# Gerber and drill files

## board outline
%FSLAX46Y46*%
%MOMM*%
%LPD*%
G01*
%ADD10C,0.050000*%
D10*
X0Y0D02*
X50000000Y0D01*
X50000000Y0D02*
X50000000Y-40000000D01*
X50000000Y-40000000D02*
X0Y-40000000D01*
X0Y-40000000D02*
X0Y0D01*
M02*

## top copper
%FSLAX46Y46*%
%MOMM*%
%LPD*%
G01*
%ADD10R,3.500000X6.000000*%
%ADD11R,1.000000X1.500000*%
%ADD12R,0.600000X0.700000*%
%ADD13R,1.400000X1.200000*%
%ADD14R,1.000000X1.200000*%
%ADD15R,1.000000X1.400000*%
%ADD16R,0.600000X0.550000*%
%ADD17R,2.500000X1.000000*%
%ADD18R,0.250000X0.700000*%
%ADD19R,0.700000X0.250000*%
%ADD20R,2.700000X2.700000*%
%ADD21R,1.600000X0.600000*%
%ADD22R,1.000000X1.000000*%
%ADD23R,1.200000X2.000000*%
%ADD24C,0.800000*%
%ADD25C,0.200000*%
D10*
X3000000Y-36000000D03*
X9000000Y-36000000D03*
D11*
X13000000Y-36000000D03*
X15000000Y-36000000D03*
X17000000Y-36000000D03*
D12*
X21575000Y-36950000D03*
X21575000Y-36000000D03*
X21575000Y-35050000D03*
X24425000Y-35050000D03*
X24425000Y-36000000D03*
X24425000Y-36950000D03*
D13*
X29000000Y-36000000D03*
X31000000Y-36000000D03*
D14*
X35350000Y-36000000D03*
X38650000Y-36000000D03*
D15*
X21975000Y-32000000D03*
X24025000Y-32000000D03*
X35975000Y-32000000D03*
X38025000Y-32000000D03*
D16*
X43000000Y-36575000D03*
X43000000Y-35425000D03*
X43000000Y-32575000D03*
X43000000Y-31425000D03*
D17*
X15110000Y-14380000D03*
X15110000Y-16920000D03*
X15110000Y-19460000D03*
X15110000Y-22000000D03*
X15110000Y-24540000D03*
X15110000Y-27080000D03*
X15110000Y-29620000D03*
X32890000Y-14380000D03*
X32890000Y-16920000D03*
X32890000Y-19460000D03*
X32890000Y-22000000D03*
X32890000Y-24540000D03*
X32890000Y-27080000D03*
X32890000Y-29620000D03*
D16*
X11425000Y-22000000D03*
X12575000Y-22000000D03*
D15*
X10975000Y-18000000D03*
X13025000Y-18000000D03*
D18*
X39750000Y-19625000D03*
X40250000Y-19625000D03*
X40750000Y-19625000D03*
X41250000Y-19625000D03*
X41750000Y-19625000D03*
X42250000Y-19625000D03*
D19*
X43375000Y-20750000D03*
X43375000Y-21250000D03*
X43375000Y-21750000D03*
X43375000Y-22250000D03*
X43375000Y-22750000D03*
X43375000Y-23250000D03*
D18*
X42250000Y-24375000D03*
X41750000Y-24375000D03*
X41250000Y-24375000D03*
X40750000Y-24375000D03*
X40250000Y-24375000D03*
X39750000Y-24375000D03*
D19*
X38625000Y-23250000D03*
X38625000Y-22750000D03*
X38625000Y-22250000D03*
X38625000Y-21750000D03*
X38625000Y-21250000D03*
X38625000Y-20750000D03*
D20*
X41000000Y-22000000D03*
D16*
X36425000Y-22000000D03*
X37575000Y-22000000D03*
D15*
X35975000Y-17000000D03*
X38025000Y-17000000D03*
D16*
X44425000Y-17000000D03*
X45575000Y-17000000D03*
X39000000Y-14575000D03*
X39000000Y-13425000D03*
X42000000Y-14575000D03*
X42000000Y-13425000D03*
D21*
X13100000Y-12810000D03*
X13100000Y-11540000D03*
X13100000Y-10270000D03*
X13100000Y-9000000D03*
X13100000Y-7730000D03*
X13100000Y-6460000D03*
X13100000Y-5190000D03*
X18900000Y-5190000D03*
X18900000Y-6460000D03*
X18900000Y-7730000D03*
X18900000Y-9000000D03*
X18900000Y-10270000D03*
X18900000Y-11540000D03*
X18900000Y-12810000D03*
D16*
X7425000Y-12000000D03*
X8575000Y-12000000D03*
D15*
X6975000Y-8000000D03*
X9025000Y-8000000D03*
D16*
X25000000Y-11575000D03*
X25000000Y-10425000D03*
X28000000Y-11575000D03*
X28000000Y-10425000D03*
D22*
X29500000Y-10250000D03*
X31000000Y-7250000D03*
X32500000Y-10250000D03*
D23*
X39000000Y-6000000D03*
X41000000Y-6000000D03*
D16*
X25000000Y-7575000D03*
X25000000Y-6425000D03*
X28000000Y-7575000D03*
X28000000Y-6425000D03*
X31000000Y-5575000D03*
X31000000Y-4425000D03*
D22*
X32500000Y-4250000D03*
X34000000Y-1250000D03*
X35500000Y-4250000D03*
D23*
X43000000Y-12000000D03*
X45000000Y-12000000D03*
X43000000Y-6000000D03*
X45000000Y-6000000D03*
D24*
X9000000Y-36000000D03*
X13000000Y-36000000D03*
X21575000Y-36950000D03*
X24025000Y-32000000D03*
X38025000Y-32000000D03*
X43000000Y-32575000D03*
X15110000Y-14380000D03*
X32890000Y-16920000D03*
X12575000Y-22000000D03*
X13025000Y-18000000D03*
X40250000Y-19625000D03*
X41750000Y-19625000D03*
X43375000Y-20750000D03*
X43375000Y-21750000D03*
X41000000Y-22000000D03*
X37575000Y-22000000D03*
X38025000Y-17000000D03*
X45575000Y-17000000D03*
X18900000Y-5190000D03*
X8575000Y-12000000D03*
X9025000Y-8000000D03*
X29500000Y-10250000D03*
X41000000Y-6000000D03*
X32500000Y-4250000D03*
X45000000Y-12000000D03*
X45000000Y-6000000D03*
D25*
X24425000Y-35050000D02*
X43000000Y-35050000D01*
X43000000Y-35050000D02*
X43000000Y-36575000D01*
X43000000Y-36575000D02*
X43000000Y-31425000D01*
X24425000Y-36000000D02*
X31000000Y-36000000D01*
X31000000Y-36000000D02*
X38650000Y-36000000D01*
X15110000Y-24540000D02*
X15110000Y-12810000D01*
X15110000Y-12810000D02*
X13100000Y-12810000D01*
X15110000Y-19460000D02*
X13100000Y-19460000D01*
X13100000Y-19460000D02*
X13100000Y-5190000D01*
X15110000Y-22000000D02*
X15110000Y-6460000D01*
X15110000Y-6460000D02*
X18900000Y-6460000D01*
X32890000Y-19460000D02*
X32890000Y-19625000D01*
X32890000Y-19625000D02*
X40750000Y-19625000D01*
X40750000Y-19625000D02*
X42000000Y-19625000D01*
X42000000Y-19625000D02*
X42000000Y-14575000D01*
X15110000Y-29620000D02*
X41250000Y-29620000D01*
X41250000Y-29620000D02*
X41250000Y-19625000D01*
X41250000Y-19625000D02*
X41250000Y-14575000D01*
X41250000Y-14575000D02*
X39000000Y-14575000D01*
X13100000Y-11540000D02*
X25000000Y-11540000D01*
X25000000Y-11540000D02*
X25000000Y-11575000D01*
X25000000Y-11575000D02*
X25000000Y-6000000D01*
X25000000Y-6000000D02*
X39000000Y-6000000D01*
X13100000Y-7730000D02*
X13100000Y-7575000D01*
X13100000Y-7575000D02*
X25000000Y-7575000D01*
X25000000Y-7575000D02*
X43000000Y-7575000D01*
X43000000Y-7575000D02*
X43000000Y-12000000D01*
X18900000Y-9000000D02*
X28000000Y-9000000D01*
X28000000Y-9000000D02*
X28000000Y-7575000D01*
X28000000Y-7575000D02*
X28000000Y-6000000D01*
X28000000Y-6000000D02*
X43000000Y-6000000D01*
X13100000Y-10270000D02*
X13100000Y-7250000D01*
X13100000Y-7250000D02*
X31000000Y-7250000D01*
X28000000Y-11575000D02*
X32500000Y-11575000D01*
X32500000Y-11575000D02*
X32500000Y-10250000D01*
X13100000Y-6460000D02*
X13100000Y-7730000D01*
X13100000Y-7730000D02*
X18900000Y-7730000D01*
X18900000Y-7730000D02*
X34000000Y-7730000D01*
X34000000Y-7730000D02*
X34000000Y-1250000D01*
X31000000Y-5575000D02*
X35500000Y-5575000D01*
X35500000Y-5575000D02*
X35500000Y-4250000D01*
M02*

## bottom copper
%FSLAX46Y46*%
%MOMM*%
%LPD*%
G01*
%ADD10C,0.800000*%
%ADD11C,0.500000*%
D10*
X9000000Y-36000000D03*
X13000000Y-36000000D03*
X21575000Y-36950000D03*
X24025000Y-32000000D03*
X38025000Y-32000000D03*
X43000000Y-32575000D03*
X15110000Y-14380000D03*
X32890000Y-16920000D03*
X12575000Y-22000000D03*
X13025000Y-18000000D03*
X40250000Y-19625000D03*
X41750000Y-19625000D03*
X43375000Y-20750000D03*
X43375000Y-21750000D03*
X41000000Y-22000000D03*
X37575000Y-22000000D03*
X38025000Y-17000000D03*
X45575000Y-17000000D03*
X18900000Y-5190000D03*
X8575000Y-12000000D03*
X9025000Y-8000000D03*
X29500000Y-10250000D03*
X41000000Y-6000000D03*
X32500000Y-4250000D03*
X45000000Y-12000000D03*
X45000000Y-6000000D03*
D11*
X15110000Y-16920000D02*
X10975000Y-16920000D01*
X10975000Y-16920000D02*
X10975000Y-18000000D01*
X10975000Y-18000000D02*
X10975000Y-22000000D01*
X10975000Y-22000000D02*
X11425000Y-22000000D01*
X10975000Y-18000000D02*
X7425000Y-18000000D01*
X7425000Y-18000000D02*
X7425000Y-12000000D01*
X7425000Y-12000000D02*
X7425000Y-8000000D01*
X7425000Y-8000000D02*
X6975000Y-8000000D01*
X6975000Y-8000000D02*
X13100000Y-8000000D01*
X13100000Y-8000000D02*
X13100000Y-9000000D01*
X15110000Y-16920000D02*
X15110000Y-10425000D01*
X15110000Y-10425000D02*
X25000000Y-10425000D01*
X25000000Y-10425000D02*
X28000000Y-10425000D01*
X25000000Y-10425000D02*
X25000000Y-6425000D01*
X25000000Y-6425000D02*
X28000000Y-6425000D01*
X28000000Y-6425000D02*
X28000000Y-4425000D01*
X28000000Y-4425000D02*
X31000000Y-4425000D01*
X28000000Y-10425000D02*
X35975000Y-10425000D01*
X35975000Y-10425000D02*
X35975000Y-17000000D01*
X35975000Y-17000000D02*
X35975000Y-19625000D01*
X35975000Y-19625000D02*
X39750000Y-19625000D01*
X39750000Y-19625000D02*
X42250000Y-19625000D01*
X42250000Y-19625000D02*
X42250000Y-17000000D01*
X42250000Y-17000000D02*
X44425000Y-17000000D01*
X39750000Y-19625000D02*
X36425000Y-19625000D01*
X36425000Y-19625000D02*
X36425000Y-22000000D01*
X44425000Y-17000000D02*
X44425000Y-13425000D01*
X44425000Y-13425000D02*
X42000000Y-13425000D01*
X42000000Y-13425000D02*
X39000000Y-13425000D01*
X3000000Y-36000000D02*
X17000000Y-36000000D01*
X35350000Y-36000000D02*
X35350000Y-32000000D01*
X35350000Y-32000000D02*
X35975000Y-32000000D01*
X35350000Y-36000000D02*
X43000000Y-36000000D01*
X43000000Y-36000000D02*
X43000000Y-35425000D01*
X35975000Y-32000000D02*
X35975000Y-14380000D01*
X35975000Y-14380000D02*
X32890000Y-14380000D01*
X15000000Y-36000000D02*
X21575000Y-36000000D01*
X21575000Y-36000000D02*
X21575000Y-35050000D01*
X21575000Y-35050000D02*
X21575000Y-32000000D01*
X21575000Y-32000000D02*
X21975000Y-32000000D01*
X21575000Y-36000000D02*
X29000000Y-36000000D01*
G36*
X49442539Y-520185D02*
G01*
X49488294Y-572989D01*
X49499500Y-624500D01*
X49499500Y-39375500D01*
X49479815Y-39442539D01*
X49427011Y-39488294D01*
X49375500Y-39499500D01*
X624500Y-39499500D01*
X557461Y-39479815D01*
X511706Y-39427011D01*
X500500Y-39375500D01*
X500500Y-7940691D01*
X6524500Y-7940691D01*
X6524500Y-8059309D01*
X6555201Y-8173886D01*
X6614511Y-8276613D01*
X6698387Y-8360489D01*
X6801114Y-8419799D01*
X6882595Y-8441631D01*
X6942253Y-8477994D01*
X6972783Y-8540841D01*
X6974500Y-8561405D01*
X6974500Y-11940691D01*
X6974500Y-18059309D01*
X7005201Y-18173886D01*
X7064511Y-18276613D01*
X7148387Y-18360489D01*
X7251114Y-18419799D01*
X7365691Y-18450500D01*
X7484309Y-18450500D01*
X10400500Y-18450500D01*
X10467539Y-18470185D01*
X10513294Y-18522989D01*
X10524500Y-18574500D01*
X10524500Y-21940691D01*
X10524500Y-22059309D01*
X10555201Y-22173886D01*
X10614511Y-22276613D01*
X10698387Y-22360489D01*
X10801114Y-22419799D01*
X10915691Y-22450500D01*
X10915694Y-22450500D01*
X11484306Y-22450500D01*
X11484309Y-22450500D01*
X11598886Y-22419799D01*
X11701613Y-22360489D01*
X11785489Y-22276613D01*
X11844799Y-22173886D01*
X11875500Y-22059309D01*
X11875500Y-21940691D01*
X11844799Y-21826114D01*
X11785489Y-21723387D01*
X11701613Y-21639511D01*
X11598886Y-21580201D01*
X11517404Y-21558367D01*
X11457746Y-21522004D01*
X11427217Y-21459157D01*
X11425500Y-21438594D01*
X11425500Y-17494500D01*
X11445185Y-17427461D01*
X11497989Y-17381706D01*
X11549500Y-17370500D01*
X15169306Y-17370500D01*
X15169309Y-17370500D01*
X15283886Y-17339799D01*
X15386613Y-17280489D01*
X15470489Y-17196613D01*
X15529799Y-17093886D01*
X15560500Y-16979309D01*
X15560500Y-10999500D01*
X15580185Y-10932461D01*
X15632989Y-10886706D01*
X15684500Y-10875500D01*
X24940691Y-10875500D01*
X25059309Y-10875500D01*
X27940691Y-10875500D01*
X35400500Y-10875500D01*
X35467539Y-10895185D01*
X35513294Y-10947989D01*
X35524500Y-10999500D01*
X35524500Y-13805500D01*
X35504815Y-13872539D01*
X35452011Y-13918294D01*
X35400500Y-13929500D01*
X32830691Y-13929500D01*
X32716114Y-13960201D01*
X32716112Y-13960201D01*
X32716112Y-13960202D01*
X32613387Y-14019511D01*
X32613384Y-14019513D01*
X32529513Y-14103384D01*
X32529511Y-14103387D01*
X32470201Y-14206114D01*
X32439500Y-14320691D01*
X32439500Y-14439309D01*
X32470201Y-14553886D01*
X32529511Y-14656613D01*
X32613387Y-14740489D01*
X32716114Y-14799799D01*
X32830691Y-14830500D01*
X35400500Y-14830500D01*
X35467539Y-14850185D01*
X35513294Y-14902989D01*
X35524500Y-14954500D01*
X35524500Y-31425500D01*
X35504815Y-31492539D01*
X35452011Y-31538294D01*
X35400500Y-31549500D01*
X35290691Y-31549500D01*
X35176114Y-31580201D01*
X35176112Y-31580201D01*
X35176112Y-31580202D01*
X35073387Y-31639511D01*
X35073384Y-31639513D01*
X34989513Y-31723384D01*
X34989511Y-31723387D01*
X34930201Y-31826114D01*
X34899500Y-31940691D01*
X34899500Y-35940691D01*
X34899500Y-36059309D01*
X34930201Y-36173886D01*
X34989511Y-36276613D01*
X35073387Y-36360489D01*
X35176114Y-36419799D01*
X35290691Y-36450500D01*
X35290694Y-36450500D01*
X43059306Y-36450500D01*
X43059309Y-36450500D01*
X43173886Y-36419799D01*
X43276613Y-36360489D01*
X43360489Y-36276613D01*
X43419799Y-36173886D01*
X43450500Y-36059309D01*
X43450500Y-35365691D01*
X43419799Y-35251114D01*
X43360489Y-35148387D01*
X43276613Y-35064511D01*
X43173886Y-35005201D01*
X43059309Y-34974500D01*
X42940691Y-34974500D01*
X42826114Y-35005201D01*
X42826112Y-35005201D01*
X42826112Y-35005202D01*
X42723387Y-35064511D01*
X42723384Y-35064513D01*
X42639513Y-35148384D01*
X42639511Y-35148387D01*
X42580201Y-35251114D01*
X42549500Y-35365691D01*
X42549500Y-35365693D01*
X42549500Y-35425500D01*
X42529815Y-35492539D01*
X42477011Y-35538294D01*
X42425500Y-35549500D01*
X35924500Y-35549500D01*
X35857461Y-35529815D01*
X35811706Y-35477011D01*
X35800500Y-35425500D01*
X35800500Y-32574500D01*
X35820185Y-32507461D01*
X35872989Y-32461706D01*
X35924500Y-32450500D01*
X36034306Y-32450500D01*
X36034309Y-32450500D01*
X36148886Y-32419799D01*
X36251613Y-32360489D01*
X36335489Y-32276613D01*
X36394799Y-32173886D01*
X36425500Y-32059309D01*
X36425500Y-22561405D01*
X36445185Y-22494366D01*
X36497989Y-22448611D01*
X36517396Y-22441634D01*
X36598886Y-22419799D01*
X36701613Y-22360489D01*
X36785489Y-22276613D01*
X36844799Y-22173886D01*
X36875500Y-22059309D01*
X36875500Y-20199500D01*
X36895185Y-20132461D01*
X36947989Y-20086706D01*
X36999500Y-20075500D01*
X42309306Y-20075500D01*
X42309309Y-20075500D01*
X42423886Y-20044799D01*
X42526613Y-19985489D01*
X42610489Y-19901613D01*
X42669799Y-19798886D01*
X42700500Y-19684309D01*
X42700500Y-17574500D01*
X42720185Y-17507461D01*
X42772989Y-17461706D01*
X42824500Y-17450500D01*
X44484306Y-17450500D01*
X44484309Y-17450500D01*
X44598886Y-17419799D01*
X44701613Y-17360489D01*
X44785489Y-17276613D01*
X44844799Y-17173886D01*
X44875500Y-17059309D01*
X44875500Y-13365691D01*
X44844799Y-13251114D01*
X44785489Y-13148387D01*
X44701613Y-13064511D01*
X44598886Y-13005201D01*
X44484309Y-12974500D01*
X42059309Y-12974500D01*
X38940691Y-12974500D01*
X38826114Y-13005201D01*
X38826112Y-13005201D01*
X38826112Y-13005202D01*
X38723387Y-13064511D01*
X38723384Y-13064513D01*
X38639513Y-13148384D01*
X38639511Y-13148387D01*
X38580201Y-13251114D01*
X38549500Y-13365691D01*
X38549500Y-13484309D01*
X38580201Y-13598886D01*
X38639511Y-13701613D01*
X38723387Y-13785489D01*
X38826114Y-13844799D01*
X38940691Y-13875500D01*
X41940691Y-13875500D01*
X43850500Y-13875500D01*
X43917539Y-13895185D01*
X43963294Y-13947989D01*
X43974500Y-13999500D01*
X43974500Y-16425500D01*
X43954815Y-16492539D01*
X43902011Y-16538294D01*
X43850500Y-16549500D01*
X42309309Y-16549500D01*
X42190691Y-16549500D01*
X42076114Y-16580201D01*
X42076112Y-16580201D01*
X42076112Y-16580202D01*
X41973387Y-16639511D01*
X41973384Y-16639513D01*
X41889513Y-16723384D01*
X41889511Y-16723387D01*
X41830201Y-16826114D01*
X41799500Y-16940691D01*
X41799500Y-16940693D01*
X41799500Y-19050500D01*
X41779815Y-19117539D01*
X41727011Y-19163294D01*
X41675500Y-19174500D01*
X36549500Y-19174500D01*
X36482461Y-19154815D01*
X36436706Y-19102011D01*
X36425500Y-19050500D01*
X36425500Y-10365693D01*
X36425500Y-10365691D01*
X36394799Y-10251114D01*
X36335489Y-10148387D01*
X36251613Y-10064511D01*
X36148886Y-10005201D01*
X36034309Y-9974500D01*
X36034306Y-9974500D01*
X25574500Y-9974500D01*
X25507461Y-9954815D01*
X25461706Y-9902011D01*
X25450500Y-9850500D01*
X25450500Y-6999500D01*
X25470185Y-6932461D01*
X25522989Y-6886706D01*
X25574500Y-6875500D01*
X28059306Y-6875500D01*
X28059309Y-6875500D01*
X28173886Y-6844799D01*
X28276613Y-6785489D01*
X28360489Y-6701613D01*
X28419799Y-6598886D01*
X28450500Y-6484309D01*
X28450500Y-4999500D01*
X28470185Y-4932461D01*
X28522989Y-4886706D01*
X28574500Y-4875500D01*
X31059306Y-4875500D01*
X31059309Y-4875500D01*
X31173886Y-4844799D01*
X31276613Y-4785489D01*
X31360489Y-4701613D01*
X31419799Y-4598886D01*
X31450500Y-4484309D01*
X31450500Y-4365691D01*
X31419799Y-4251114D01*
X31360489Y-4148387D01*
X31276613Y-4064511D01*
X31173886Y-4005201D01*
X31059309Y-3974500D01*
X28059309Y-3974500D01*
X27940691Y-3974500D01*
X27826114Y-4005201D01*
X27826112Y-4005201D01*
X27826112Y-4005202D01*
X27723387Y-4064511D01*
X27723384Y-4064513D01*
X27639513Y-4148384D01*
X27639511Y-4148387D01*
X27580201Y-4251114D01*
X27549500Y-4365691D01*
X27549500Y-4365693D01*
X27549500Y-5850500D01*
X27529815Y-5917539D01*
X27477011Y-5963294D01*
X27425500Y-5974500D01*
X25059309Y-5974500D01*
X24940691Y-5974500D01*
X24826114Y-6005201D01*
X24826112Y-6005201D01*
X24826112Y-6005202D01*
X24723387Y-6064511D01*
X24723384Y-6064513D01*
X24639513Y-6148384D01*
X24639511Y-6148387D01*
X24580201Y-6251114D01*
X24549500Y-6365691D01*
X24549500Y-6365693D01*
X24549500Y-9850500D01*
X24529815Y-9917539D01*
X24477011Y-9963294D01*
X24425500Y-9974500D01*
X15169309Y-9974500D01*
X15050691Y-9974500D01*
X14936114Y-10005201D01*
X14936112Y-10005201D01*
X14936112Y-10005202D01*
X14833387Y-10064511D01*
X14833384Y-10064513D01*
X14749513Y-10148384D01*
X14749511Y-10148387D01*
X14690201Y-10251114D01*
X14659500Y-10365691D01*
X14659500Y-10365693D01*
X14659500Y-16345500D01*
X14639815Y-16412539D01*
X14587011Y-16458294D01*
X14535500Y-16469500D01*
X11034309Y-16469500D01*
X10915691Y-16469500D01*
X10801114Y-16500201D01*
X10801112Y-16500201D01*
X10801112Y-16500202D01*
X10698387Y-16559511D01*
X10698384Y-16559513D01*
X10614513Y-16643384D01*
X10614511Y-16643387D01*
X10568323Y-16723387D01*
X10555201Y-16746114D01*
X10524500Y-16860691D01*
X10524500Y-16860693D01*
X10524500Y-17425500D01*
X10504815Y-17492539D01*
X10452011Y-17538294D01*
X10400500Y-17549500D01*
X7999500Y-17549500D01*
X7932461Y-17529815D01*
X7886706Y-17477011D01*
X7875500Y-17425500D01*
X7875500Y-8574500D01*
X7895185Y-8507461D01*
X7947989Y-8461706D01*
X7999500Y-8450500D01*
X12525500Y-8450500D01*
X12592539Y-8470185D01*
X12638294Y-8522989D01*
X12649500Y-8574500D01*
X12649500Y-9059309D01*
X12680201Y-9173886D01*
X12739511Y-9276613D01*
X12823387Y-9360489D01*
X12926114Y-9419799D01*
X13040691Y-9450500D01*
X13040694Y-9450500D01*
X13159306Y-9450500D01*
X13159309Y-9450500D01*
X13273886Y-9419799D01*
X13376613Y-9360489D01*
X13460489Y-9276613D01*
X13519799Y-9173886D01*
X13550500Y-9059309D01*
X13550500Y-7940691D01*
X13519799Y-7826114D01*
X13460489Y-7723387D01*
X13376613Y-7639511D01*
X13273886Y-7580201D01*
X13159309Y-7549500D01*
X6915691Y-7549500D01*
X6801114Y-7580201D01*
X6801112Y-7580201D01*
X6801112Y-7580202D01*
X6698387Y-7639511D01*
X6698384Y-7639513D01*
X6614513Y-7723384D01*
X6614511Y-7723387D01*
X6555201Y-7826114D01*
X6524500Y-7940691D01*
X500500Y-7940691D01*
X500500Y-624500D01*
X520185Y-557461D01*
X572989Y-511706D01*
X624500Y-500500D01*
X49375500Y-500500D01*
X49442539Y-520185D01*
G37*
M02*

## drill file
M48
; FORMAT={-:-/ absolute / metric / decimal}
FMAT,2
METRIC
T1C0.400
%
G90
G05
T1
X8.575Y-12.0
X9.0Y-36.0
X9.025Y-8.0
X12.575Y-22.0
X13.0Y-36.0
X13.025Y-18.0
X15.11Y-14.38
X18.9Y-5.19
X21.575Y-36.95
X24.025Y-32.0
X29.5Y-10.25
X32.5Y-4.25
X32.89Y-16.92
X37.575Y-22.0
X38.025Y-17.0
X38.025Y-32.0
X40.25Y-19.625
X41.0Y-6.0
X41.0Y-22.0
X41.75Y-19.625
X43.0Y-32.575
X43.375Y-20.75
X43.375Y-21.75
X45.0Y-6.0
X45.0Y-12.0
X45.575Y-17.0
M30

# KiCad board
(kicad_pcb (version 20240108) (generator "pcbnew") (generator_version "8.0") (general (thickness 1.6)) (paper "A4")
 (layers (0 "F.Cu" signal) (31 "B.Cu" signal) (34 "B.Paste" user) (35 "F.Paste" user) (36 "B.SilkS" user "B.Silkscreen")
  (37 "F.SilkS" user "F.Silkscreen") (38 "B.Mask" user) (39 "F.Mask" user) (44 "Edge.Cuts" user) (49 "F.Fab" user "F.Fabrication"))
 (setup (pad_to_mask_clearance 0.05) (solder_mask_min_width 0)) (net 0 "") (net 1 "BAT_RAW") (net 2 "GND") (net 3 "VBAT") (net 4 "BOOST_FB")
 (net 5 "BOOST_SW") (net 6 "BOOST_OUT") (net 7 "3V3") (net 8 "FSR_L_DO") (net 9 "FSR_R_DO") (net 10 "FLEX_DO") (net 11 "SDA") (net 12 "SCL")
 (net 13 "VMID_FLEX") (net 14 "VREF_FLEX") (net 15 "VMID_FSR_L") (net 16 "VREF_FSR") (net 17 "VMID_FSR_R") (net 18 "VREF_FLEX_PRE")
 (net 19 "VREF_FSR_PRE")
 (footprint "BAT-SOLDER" (layer "F.Cu") (at 6.0000 36.0000 0)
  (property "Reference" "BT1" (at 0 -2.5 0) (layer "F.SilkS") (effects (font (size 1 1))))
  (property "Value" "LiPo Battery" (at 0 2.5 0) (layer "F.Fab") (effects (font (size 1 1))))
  (pad "+" smd rect (at -3.0000 0.0000) (size 3.5000 6.0000) (layers "F.Cu" "F.Paste" "F.Mask") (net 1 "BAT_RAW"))
  (pad "-" smd rect (at 3.0000 0.0000) (size 3.5000 6.0000) (layers "F.Cu" "F.Paste" "F.Mask") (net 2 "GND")))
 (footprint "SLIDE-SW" (layer "F.Cu") (at 15.0000 36.0000 0)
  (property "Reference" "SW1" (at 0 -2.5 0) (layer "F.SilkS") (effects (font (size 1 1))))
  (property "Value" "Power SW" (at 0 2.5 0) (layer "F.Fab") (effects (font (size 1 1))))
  (pad "1" smd rect (at -2.0000 0.0000) (size 1.0000 1.5000) (layers "F.Cu" "F.Paste" "F.Mask") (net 2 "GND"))
  (pad "2" smd rect (at 0.0000 0.0000) (size 1.0000 1.5000) (layers "F.Cu" "F.Paste" "F.Mask") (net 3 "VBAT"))
  (pad "3" smd rect (at 2.0000 0.0000) (size 1.0000 1.5000) (layers "F.Cu" "F.Paste" "F.Mask") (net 1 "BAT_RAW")))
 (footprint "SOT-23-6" (layer "F.Cu") (at 23.0000 36.0000 0)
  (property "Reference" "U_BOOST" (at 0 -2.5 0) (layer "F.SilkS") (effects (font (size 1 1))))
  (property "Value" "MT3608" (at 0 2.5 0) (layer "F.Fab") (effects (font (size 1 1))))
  (pad "1" smd rect (at -1.4250 0.9500) (size 0.6000 0.7000) (layers "F.Cu" "F.Paste" "F.Mask") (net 2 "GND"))
  (pad "2" smd rect (at -1.4250 0.0000) (size 0.6000 0.7000) (layers "F.Cu" "F.Paste" "F.Mask") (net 3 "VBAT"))
  (pad "3" smd rect (at -1.4250 -0.9500) (size 0.6000 0.7000) (layers "F.Cu" "F.Paste" "F.Mask") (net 3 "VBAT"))
  (pad "4" smd rect (at 1.4250 -0.9500) (size 0.6000 0.7000) (layers "F.Cu" "F.Paste" "F.Mask") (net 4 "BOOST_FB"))
  (pad "5" smd rect (at 1.4250 0.0000) (size 0.6000 0.7000) (layers "F.Cu" "F.Paste" "F.Mask") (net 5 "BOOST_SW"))
  (pad "6" smd rect (at 1.4250 0.9500) (size 0.6000 0.7000) (layers "F.Cu" "F.Paste" "F.Mask")))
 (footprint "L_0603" (layer "F.Cu") (at 30.0000 36.0000 0)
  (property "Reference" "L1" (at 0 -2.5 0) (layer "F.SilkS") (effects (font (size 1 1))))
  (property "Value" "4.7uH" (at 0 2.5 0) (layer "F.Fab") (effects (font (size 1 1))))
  (pad "1" smd rect (at -1.0000 0.0000) (size 1.4000 1.2000) (layers "F.Cu" "F.Paste" "F.Mask") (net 3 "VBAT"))
  (pad "2" smd rect (at 1.0000 0.0000) (size 1.4000 1.2000) (layers "F.Cu" "F.Paste" "F.Mask") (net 5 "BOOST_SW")))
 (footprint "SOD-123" (layer "F.Cu") (at 37.0000 36.0000 0)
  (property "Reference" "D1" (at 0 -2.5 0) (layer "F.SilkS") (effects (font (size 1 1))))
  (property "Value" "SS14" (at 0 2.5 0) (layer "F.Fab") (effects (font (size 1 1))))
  (pad "K" smd rect (at -1.6500 0.0000) (size 1.0000 1.2000) (layers "F.Cu" "F.Paste" "F.Mask") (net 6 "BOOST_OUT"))
  (pad "A" smd rect (at 1.6500 0.0000) (size 1.0000 1.2000) (layers "F.Cu" "F.Paste" "F.Mask") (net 5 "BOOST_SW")))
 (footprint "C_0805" (layer "F.Cu") (at 23.0000 32.0000 0)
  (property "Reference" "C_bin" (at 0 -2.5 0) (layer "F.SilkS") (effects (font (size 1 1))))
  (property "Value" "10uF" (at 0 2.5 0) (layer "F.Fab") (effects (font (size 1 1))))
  (pad "1" smd rect (at -1.0250 0.0000) (size 1.0000 1.4000) (layers "F.Cu" "F.Paste" "F.Mask") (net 3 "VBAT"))
  (pad "2" smd rect (at 1.0250 0.0000) (size 1.0000 1.4000) (layers "F.Cu" "F.Paste" "F.Mask") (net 2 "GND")))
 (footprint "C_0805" (layer "F.Cu") (at 37.0000 32.0000 0)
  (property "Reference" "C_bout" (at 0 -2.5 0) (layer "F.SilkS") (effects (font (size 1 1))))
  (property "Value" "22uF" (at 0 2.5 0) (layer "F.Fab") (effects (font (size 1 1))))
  (pad "1" smd rect (at -1.0250 0.0000) (size 1.0000 1.4000) (layers "F.Cu" "F.Paste" "F.Mask") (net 6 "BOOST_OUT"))
  (pad "2" smd rect (at 1.0250 0.0000) (size 1.0000 1.4000) (layers "F.Cu" "F.Paste" "F.Mask") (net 2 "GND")))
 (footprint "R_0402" (layer "F.Cu") (at 43.0000 36.0000 90)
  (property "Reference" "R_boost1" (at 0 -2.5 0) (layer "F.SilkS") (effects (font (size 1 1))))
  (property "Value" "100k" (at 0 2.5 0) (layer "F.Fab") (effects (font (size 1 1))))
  (pad "1" smd rect (at -0.5750 0.0000) (size 0.6000 0.5500) (layers "F.Cu" "F.Paste" "F.Mask") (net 6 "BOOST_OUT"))
  (pad "2" smd rect (at 0.5750 0.0000) (size 0.6000 0.5500) (layers "F.Cu" "F.Paste" "F.Mask") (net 4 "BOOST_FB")))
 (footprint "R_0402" (layer "F.Cu") (at 43.0000 32.0000 90)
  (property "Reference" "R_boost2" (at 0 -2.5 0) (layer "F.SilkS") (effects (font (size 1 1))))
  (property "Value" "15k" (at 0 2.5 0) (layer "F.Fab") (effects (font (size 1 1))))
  (pad "1" smd rect (at -0.5750 0.0000) (size 0.6000 0.5500) (layers "F.Cu" "F.Paste" "F.Mask") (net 4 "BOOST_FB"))
  (pad "2" smd rect (at 0.5750 0.0000) (size 0.6000 0.5500) (layers "F.Cu" "F.Paste" "F.Mask") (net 2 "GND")))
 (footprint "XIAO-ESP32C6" (layer "F.Cu") (at 24.0000 22.0000 0)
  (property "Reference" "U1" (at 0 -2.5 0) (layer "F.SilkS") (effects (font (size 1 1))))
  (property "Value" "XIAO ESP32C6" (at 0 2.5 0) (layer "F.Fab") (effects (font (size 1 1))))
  (pad "1" smd rect (at -8.8900 -7.6200) (size 2.5000 1.0000) (layers "F.Cu" "F.Paste" "F.Mask") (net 2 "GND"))
  (pad "2" smd rect (at -8.8900 -5.0800) (size 2.5000 1.0000) (layers "F.Cu" "F.Paste" "F.Mask") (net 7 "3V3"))
  (pad "3" smd rect (at -8.8900 -2.5400) (size 2.5000 1.0000) (layers "F.Cu" "F.Paste" "F.Mask") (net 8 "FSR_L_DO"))
  (pad "4" smd rect (at -8.8900 0.0000) (size 2.5000 1.0000) (layers "F.Cu" "F.Paste" "F.Mask") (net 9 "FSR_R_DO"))
  (pad "5" smd rect (at -8.8900 2.5400) (size 2.5000 1.0000) (layers "F.Cu" "F.Paste" "F.Mask") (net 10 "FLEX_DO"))
  (pad "6" smd rect (at -8.8900 5.0800) (size 2.5000 1.0000) (layers "F.Cu" "F.Paste" "F.Mask"))
  (pad "7" smd rect (at -8.8900 7.6200) (size 2.5000 1.0000) (layers "F.Cu" "F.Paste" "F.Mask") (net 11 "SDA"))
  (pad "8" smd rect (at 8.8900 -7.6200) (size 2.5000 1.0000) (layers "F.Cu" "F.Paste" "F.Mask") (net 6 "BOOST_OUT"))
  (pad "9" smd rect (at 8.8900 -5.0800) (size 2.5000 1.0000) (layers "F.Cu" "F.Paste" "F.Mask") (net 2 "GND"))
  (pad "10" smd rect (at 8.8900 -2.5400) (size 2.5000 1.0000) (layers "F.Cu" "F.Paste" "F.Mask") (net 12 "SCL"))
  (pad "11" smd rect (at 8.8900 0.0000) (size 2.5000 1.0000) (layers "F.Cu" "F.Paste" "F.Mask"))
  (pad "12" smd rect (at 8.8900 2.5400) (size 2.5000 1.0000) (layers "F.Cu" "F.Paste" "F.Mask"))
  (pad "13" smd rect (at 8.8900 5.0800) (size 2.5000 1.0000) (layers "F.Cu" "F.Paste" "F.Mask"))
  (pad "14" smd rect (at 8.8900 7.6200) (size 2.5000 1.0000) (layers "F.Cu" "F.Paste" "F.Mask")))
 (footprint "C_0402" (layer "F.Cu") (at 12.0000 22.0000 0)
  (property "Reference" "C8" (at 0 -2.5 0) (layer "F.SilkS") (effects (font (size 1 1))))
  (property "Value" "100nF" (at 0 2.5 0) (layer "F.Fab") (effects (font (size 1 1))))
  (pad "1" smd rect (at -0.5750 0.0000) (size 0.6000 0.5500) (layers "F.Cu" "F.Paste" "F.Mask") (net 7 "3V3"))
  (pad "2" smd rect (at 0.5750 0.0000) (size 0.6000 0.5500) (layers "F.Cu" "F.Paste" "F.Mask") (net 2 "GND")))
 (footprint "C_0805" (layer "F.Cu") (at 12.0000 18.0000 0)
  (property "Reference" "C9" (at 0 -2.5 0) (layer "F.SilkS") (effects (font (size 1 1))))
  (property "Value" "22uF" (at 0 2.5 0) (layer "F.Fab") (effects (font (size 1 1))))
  (pad "1" smd rect (at -1.0250 0.0000) (size 1.0000 1.4000) (layers "F.Cu" "F.Paste" "F.Mask") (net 7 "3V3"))
  (pad "2" smd rect (at 1.0250 0.0000) (size 1.0000 1.4000) (layers "F.Cu" "F.Paste" "F.Mask") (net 2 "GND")))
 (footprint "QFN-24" (layer "F.Cu") (at 41.0000 22.0000 0)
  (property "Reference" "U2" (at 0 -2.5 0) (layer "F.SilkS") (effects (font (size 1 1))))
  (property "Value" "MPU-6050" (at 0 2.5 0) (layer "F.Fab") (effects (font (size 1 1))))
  (pad "1" smd rect (at -1.2500 -2.3750) (size 0.2500 0.7000) (layers "F.Cu" "F.Paste" "F.Mask") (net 7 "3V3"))
  (pad "2" smd rect (at -0.7500 -2.3750) (size 0.2500 0.7000) (layers "F.Cu" "F.Paste" "F.Mask") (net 2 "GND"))
  (pad "3" smd rect (at -0.2500 -2.3750) (size 0.2500 0.7000) (layers "F.Cu" "F.Paste" "F.Mask") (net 12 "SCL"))
  (pad "4" smd rect (at 0.2500 -2.3750) (size 0.2500 0.7000) (layers "F.Cu" "F.Paste" "F.Mask") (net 11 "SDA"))
  (pad "5" smd rect (at 0.7500 -2.3750) (size 0.2500 0.7000) (layers "F.Cu" "F.Paste" "F.Mask") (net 2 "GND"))
  (pad "6" smd rect (at 1.2500 -2.3750) (size 0.2500 0.7000) (layers "F.Cu" "F.Paste" "F.Mask") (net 7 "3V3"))
  (pad "7" smd rect (at 2.3750 -1.2500) (size 0.7000 0.2500) (layers "F.Cu" "F.Paste" "F.Mask") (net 2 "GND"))
  (pad "8" smd rect (at 2.3750 -0.7500) (size 0.7000 0.2500) (layers "F.Cu" "F.Paste" "F.Mask"))
  (pad "9" smd rect (at 2.3750 -0.2500) (size 0.7000 0.2500) (layers "F.Cu" "F.Paste" "F.Mask") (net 2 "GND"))
  (pad "10" smd rect (at 2.3750 0.2500) (size 0.7000 0.2500) (layers "F.Cu" "F.Paste" "F.Mask"))
  (pad "11" smd rect (at 2.3750 0.7500) (size 0.7000 0.2500) (layers "F.Cu" "F.Paste" "F.Mask"))
  (pad "12" smd rect (at 2.3750 1.2500) (size 0.7000 0.2500) (layers "F.Cu" "F.Paste" "F.Mask"))
  (pad "13" smd rect (at 1.2500 2.3750) (size 0.2500 0.7000) (layers "F.Cu" "F.Paste" "F.Mask"))
  (pad "14" smd rect (at 0.7500 2.3750) (size 0.2500 0.7000) (layers "F.Cu" "F.Paste" "F.Mask"))
  (pad "15" smd rect (at 0.2500 2.3750) (size 0.2500 0.7000) (layers "F.Cu" "F.Paste" "F.Mask"))
  (pad "16" smd rect (at -0.2500 2.3750) (size 0.2500 0.7000) (layers "F.Cu" "F.Paste" "F.Mask"))
  (pad "17" smd rect (at -0.7500 2.3750) (size 0.2500 0.7000) (layers "F.Cu" "F.Paste" "F.Mask"))
  (pad "18" smd rect (at -1.2500 2.3750) (size 0.2500 0.7000) (layers "F.Cu" "F.Paste" "F.Mask"))
  (pad "19" smd rect (at -2.3750 1.2500) (size 0.7000 0.2500) (layers "F.Cu" "F.Paste" "F.Mask"))
  (pad "20" smd rect (at -2.3750 0.7500) (size 0.7000 0.2500) (layers "F.Cu" "F.Paste" "F.Mask"))
  (pad "21" smd rect (at -2.3750 0.2500) (size 0.7000 0.2500) (layers "F.Cu" "F.Paste" "F.Mask"))
  (pad "22" smd rect (at -2.3750 -0.2500) (size 0.7000 0.2500) (layers "F.Cu" "F.Paste" "F.Mask"))
  (pad "23" smd rect (at -2.3750 -0.7500) (size 0.7000 0.2500) (layers "F.Cu" "F.Paste" "F.Mask"))
  (pad "24" smd rect (at -2.3750 -1.2500) (size 0.7000 0.2500) (layers "F.Cu" "F.Paste" "F.Mask"))
  (pad "25" smd rect (at 0.0000 0.0000) (size 2.7000 2.7000) (layers "F.Cu" "F.Paste" "F.Mask") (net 2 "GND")))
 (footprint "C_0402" (layer "F.Cu") (at 37.0000 22.0000 0)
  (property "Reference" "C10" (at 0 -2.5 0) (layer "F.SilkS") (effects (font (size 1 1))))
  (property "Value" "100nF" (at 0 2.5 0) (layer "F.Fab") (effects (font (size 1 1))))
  (pad "1" smd rect (at -0.5750 0.0000) (size 0.6000 0.5500) (layers "F.Cu" "F.Paste" "F.Mask") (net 7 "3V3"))
  (pad "2" smd rect (at 0.5750 0.0000) (size 0.6000 0.5500) (layers "F.Cu" "F.Paste" "F.Mask") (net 2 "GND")))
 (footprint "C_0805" (layer "F.Cu") (at 37.0000 17.0000 0)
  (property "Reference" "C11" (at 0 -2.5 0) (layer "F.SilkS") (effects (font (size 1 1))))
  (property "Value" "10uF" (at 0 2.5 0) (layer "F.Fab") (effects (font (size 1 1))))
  (pad "1" smd rect (at -1.0250 0.0000) (size 1.0000 1.4000) (layers "F.Cu" "F.Paste" "F.Mask") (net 7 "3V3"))
  (pad "2" smd rect (at 1.0250 0.0000) (size 1.0000 1.4000) (layers "F.Cu" "F.Paste" "F.Mask") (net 2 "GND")))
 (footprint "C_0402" (layer "F.Cu") (at 45.0000 17.0000 0)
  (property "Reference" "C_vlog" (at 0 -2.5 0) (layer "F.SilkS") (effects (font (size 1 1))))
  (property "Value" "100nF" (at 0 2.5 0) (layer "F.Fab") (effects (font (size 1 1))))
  (pad "1" smd rect (at -0.5750 0.0000) (size 0.6000 0.5500) (layers "F.Cu" "F.Paste" "F.Mask") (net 7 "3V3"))
  (pad "2" smd rect (at 0.5750 0.0000) (size 0.6000 0.5500) (layers "F.Cu" "F.Paste" "F.Mask") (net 2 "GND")))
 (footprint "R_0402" (layer "F.Cu") (at 39.0000 14.0000 90)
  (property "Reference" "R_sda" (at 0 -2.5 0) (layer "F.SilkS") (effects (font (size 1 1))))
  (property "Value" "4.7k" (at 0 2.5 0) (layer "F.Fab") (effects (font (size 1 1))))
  (pad "1" smd rect (at -0.5750 0.0000) (size 0.6000 0.5500) (layers "F.Cu" "F.Paste" "F.Mask") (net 7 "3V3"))
  (pad "2" smd rect (at 0.5750 0.0000) (size 0.6000 0.5500) (layers "F.Cu" "F.Paste" "F.Mask") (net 11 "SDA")))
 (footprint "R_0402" (layer "F.Cu") (at 42.0000 14.0000 90)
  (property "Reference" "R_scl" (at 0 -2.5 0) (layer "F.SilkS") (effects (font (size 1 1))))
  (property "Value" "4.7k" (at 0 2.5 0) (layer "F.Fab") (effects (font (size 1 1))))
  (pad "1" smd rect (at -0.5750 0.0000) (size 0.6000 0.5500) (layers "F.Cu" "F.Paste" "F.Mask") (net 7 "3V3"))
  (pad "2" smd rect (at 0.5750 0.0000) (size 0.6000 0.5500) (layers "F.Cu" "F.Paste" "F.Mask") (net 12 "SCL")))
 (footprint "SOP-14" (layer "F.Cu") (at 16.0000 9.0000 0)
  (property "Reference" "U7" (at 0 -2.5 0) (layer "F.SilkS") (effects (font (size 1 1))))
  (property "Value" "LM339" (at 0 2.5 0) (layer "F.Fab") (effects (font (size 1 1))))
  (pad "1" smd rect (at -2.9000 3.8100) (size 1.6000 0.6000) (layers "F.Cu" "F.Paste" "F.Mask") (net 10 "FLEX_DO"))
  (pad "2" smd rect (at -2.9000 2.5400) (size 1.6000 0.6000) (layers "F.Cu" "F.Paste" "F.Mask") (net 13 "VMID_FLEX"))
  (pad "3" smd rect (at -2.9000 1.2700) (size 1.6000 0.6000) (layers "F.Cu" "F.Paste" "F.Mask") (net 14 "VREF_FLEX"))
  (pad "4" smd rect (at -2.9000 0.0000) (size 1.6000 0.6000) (layers "F.Cu" "F.Paste" "F.Mask") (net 7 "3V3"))
  (pad "5" smd rect (at -2.9000 -1.2700) (size 1.6000 0.6000) (layers "F.Cu" "F.Paste" "F.Mask") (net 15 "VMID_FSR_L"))
  (pad "6" smd rect (at -2.9000 -2.5400) (size 1.6000 0.6000) (layers "F.Cu" "F.Paste" "F.Mask") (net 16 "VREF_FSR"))
  (pad "7" smd rect (at -2.9000 -3.8100) (size 1.6000 0.6000) (layers "F.Cu" "F.Paste" "F.Mask") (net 8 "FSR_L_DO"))
  (pad "8" smd rect (at 2.9000 -3.8100) (size 1.6000 0.6000) (layers "F.Cu" "F.Paste" "F.Mask") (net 2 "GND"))
  (pad "9" smd rect (at 2.9000 -2.5400) (size 1.6000 0.6000) (layers "F.Cu" "F.Paste" "F.Mask") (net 9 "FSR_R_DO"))
  (pad "10" smd rect (at 2.9000 -1.2700) (size 1.6000 0.6000) (layers "F.Cu" "F.Paste" "F.Mask") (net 16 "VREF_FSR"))
  (pad "11" smd rect (at 2.9000 -0.0000) (size 1.6000 0.6000) (layers "F.Cu" "F.Paste" "F.Mask") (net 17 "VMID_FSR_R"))
  (pad "12" smd rect (at 2.9000 1.2700) (size 1.6000 0.6000) (layers "F.Cu" "F.Paste" "F.Mask"))
  (pad "13" smd rect (at 2.9000 2.5400) (size 1.6000 0.6000) (layers "F.Cu" "F.Paste" "F.Mask"))
  (pad "14" smd rect (at 2.9000 3.8100) (size 1.6000 0.6000) (layers "F.Cu" "F.Paste" "F.Mask")))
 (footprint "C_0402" (layer "F.Cu") (at 8.0000 12.0000 0)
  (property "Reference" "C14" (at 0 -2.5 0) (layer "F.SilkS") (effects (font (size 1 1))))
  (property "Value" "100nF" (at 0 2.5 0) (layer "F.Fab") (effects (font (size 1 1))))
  (pad "1" smd rect (at -0.5750 0.0000) (size 0.6000 0.5500) (layers "F.Cu" "F.Paste" "F.Mask") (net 7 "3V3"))
  (pad "2" smd rect (at 0.5750 0.0000) (size 0.6000 0.5500) (layers "F.Cu" "F.Paste" "F.Mask") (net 2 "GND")))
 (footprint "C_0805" (layer "F.Cu") (at 8.0000 8.0000 0)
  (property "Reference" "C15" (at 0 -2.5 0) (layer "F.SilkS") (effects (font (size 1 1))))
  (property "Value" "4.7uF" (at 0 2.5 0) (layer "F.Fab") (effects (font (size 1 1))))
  (pad "1" smd rect (at -1.0250 0.0000) (size 1.0000 1.4000) (layers "F.Cu" "F.Paste" "F.Mask") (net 7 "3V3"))
  (pad "2" smd rect (at 1.0250 0.0000) (size 1.0000 1.4000) (layers "F.Cu" "F.Paste" "F.Mask") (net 2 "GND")))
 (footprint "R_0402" (layer "F.Cu") (at 25.0000 11.0000 90)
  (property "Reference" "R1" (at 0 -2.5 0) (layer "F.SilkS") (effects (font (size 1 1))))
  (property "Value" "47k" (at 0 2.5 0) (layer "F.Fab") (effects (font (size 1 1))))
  (pad "1" smd rect (at -0.5750 0.0000) (size 0.6000 0.5500) (layers "F.Cu" "F.Paste" "F.Mask") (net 7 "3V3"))
  (pad "2" smd rect (at 0.5750 0.0000) (size 0.6000 0.5500) (layers "F.Cu" "F.Paste" "F.Mask") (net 13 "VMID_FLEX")))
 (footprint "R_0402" (layer "F.Cu") (at 28.0000 11.0000 90)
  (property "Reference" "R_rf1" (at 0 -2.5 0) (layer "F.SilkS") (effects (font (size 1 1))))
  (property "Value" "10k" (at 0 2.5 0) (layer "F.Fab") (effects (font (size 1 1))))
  (pad "1" smd rect (at -0.5750 0.0000) (size 0.6000 0.5500) (layers "F.Cu" "F.Paste" "F.Mask") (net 7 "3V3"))
  (pad "2" smd rect (at 0.5750 0.0000) (size 0.6000 0.5500) (layers "F.Cu" "F.Paste" "F.Mask") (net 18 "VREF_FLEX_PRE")))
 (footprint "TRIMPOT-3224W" (layer "F.Cu") (at 31.0000 9.0000 0)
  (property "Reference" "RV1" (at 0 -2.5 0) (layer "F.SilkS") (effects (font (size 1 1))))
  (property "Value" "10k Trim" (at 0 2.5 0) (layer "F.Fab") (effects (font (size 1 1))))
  (pad "1" smd rect (at -1.5000 1.2500) (size 1.0000 1.0000) (layers "F.Cu" "F.Paste" "F.Mask") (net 2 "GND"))
  (pad "W" smd rect (at 0.0000 -1.7500) (size 1.0000 1.0000) (layers "F.Cu" "F.Paste" "F.Mask") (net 14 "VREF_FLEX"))
  (pad "3" smd rect (at 1.5000 1.2500) (size 1.0000 1.0000) (layers "F.Cu" "F.Paste" "F.Mask") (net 18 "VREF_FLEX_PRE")))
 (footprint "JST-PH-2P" (layer "F.Cu") (at 40.0000 6.0000 0)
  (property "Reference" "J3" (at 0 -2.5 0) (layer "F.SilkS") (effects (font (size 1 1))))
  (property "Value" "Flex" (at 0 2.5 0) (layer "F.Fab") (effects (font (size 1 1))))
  (pad "1" smd rect (at -1.0000 0.0000) (size 1.2000 2.0000) (layers "F.Cu" "F.Paste" "F.Mask") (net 13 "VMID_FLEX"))
  (pad "2" smd rect (at 1.0000 0.0000) (size 1.2000 2.0000) (layers "F.Cu" "F.Paste" "F.Mask") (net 2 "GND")))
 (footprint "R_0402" (layer "F.Cu") (at 25.0000 7.0000 90)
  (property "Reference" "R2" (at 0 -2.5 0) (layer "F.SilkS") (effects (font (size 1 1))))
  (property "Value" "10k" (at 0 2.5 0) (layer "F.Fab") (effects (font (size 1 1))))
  (pad "1" smd rect (at -0.5750 0.0000) (size 0.6000 0.5500) (layers "F.Cu" "F.Paste" "F.Mask") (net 7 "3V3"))
  (pad "2" smd rect (at 0.5750 0.0000) (size 0.6000 0.5500) (layers "F.Cu" "F.Paste" "F.Mask") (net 15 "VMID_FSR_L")))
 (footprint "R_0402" (layer "F.Cu") (at 28.0000 7.0000 90)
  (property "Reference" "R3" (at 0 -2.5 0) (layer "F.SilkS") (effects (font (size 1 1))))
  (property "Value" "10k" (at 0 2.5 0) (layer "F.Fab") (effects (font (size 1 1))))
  (pad "1" smd rect (at -0.5750 0.0000) (size 0.6000 0.5500) (layers "F.Cu" "F.Paste" "F.Mask") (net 7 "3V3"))
  (pad "2" smd rect (at 0.5750 0.0000) (size 0.6000 0.5500) (layers "F.Cu" "F.Paste" "F.Mask") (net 17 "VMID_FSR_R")))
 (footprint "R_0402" (layer "F.Cu") (at 31.0000 5.0000 90)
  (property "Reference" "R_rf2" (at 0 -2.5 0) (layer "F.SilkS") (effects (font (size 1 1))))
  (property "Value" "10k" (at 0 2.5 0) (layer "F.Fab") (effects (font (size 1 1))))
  (pad "1" smd rect (at -0.5750 0.0000) (size 0.6000 0.5500) (layers "F.Cu" "F.Paste" "F.Mask") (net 7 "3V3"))
  (pad "2" smd rect (at 0.5750 0.0000) (size 0.6000 0.5500) (layers "F.Cu" "F.Paste" "F.Mask") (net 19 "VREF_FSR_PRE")))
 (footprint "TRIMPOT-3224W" (layer "F.Cu") (at 34.0000 3.0000 0)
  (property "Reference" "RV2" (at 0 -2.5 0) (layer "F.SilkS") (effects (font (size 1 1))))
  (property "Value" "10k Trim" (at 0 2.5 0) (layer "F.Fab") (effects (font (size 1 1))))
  (pad "1" smd rect (at -1.5000 1.2500) (size 1.0000 1.0000) (layers "F.Cu" "F.Paste" "F.Mask") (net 2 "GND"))
  (pad "W" smd rect (at 0.0000 -1.7500) (size 1.0000 1.0000) (layers "F.Cu" "F.Paste" "F.Mask") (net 16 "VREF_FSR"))
  (pad "3" smd rect (at 1.5000 1.2500) (size 1.0000 1.0000) (layers "F.Cu" "F.Paste" "F.Mask") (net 19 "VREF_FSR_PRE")))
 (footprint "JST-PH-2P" (layer "F.Cu") (at 44.0000 12.0000 0)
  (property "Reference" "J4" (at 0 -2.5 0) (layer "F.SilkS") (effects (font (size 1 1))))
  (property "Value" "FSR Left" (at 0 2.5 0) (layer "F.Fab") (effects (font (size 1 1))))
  (pad "1" smd rect (at -1.0000 0.0000) (size 1.2000 2.0000) (layers "F.Cu" "F.Paste" "F.Mask") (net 15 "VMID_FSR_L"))
  (pad "2" smd rect (at 1.0000 0.0000) (size 1.2000 2.0000) (layers "F.Cu" "F.Paste" "F.Mask") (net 2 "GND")))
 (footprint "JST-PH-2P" (layer "F.Cu") (at 44.0000 6.0000 0)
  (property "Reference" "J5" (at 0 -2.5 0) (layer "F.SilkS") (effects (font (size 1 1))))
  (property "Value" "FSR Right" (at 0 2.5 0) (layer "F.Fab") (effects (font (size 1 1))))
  (pad "1" smd rect (at -1.0000 0.0000) (size 1.2000 2.0000) (layers "F.Cu" "F.Paste" "F.Mask") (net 17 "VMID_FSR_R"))
  (pad "2" smd rect (at 1.0000 0.0000) (size 1.2000 2.0000) (layers "F.Cu" "F.Paste" "F.Mask") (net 2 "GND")))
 (segment (start 15.1100 16.9200) (end 10.9750 16.9200) (width 0.5) (layer "B.Cu") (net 7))
 (segment (start 10.9750 16.9200) (end 10.9750 18.0000) (width 0.5) (layer "B.Cu") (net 7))
 (segment (start 10.9750 18.0000) (end 10.9750 22.0000) (width 0.5) (layer "B.Cu") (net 7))
 (segment (start 10.9750 22.0000) (end 11.4250 22.0000) (width 0.5) (layer "B.Cu") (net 7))
 (segment (start 10.9750 18.0000) (end 7.4250 18.0000) (width 0.5) (layer "B.Cu") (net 7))
 (segment (start 7.4250 18.0000) (end 7.4250 12.0000) (width 0.5) (layer "B.Cu") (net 7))
 (segment (start 7.4250 12.0000) (end 7.4250 8.0000) (width 0.5) (layer "B.Cu") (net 7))
 (segment (start 7.4250 8.0000) (end 6.9750 8.0000) (width 0.5) (layer "B.Cu") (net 7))
 (segment (start 6.9750 8.0000) (end 13.1000 8.0000) (width 0.5) (layer "B.Cu") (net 7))
 (segment (start 13.1000 8.0000) (end 13.1000 9.0000) (width 0.5) (layer "B.Cu") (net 7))
 (segment (start 15.1100 16.9200) (end 15.1100 10.4250) (width 0.5) (layer "B.Cu") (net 7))
 (segment (start 15.1100 10.4250) (end 25.0000 10.4250) (width 0.5) (layer "B.Cu") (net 7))
 (segment (start 25.0000 10.4250) (end 28.0000 10.4250) (width 0.5) (layer "B.Cu") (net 7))
 (segment (start 25.0000 10.4250) (end 25.0000 6.4250) (width 0.5) (layer "B.Cu") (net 7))
 (segment (start 25.0000 6.4250) (end 28.0000 6.4250) (width 0.5) (layer "B.Cu") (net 7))
 (segment (start 28.0000 6.4250) (end 28.0000 4.4250) (width 0.5) (layer "B.Cu") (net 7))
 (segment (start 28.0000 4.4250) (end 31.0000 4.4250) (width 0.5) (layer "B.Cu") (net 7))
 (segment (start 28.0000 10.4250) (end 35.9750 10.4250) (width 0.5) (layer "B.Cu") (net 7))
 (segment (start 35.9750 10.4250) (end 35.9750 17.0000) (width 0.5) (layer "B.Cu") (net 7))
 (segment (start 35.9750 17.0000) (end 35.9750 19.6250) (width 0.5) (layer "B.Cu") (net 7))
 (segment (start 35.9750 19.6250) (end 39.7500 19.6250) (width 0.5) (layer "B.Cu") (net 7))
 (segment (start 39.7500 19.6250) (end 42.2500 19.6250) (width 0.5) (layer "B.Cu") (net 7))
 (segment (start 42.2500 19.6250) (end 42.2500 17.0000) (width 0.5) (layer "B.Cu") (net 7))
 (segment (start 42.2500 17.0000) (end 44.4250 17.0000) (width 0.5) (layer "B.Cu") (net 7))
 (segment (start 39.7500 19.6250) (end 36.4250 19.6250) (width 0.5) (layer "B.Cu") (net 7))
 (segment (start 36.4250 19.6250) (end 36.4250 22.0000) (width 0.5) (layer "B.Cu") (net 7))
 (segment (start 44.4250 17.0000) (end 44.4250 13.4250) (width 0.5) (layer "B.Cu") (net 7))
 (segment (start 44.4250 13.4250) (end 42.0000 13.4250) (width 0.5) (layer "B.Cu") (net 7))
 (segment (start 42.0000 13.4250) (end 39.0000 13.4250) (width 0.5) (layer "B.Cu") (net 7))
 (segment (start 3.0000 36.0000) (end 17.0000 36.0000) (width 0.5) (layer "B.Cu") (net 1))
 (segment (start 24.4250 35.0500) (end 43.0000 35.0500) (width 0.2) (layer "F.Cu") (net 4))
 (segment (start 43.0000 35.0500) (end 43.0000 36.5750) (width 0.2) (layer "F.Cu") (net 4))
 (segment (start 43.0000 36.5750) (end 43.0000 31.4250) (width 0.2) (layer "F.Cu") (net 4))
 (segment (start 35.3500 36.0000) (end 35.3500 32.0000) (width 0.5) (layer "B.Cu") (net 6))
 (segment (start 35.3500 32.0000) (end 35.9750 32.0000) (width 0.5) (layer "B.Cu") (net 6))
 (segment (start 35.3500 36.0000) (end 43.0000 36.0000) (width 0.5) (layer "B.Cu") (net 6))
 (segment (start 43.0000 36.0000) (end 43.0000 35.4250) (width 0.5) (layer "B.Cu") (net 6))
 (segment (start 35.9750 32.0000) (end 35.9750 14.3800) (width 0.5) (layer "B.Cu") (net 6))
 (segment (start 35.9750 14.3800) (end 32.8900 14.3800) (width 0.5) (layer "B.Cu") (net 6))
 (segment (start 24.4250 36.0000) (end 31.0000 36.0000) (width 0.2) (layer "F.Cu") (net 5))
 (segment (start 31.0000 36.0000) (end 38.6500 36.0000) (width 0.2) (layer "F.Cu") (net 5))
 (segment (start 15.1100 24.5400) (end 15.1100 12.8100) (width 0.2) (layer "F.Cu") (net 10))
 (segment (start 15.1100 12.8100) (end 13.1000 12.8100) (width 0.2) (layer "F.Cu") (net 10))
 (segment (start 15.1100 19.4600) (end 13.1000 19.4600) (width 0.2) (layer "F.Cu") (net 8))
 (segment (start 13.1000 19.4600) (end 13.1000 5.1900) (width 0.2) (layer "F.Cu") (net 8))
 (segment (start 15.1100 22.0000) (end 15.1100 6.4600) (width 0.2) (layer "F.Cu") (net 9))
 (segment (start 15.1100 6.4600) (end 18.9000 6.4600) (width 0.2) (layer "F.Cu") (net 9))
 (segment (start 32.8900 19.4600) (end 32.8900 19.6250) (width 0.2) (layer "F.Cu") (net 12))
 (segment (start 32.8900 19.6250) (end 40.7500 19.6250) (width 0.2) (layer "F.Cu") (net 12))
 (segment (start 40.7500 19.6250) (end 42.0000 19.6250) (width 0.2) (layer "F.Cu") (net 12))
 (segment (start 42.0000 19.6250) (end 42.0000 14.5750) (width 0.2) (layer "F.Cu") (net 12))
 (segment (start 15.1100 29.6200) (end 41.2500 29.6200) (width 0.2) (layer "F.Cu") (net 11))
 (segment (start 41.2500 29.6200) (end 41.2500 19.6250) (width 0.2) (layer "F.Cu") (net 11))
 (segment (start 41.2500 19.6250) (end 41.2500 14.5750) (width 0.2) (layer "F.Cu") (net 11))
 (segment (start 41.2500 14.5750) (end 39.0000 14.5750) (width 0.2) (layer "F.Cu") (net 11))
 (segment (start 15.0000 36.0000) (end 21.5750 36.0000) (width 0.5) (layer "B.Cu") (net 3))
 (segment (start 21.5750 36.0000) (end 21.5750 35.0500) (width 0.5) (layer "B.Cu") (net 3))
 (segment (start 21.5750 35.0500) (end 21.5750 32.0000) (width 0.5) (layer "B.Cu") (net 3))
 (segment (start 21.5750 32.0000) (end 21.9750 32.0000) (width 0.5) (layer "B.Cu") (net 3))
 (segment (start 21.5750 36.0000) (end 29.0000 36.0000) (width 0.5) (layer "B.Cu") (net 3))
 (segment (start 13.1000 11.5400) (end 25.0000 11.5400) (width 0.2) (layer "F.Cu") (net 13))
 (segment (start 25.0000 11.5400) (end 25.0000 11.5750) (width 0.2) (layer "F.Cu") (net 13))
 (segment (start 25.0000 11.5750) (end 25.0000 6.0000) (width 0.2) (layer "F.Cu") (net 13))
 (segment (start 25.0000 6.0000) (end 39.0000 6.0000) (width 0.2) (layer "F.Cu") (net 13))
 (segment (start 13.1000 7.7300) (end 13.1000 7.5750) (width 0.2) (layer "F.Cu") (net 15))
 (segment (start 13.1000 7.5750) (end 25.0000 7.5750) (width 0.2) (layer "F.Cu") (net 15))
 (segment (start 25.0000 7.5750) (end 43.0000 7.5750) (width 0.2) (layer "F.Cu") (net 15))
 (segment (start 43.0000 7.5750) (end 43.0000 12.0000) (width 0.2) (layer "F.Cu") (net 15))
 (segment (start 18.9000 9.0000) (end 28.0000 9.0000) (width 0.2) (layer "F.Cu") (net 17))
 (segment (start 28.0000 9.0000) (end 28.0000 7.5750) (width 0.2) (layer "F.Cu") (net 17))
 (segment (start 28.0000 7.5750) (end 28.0000 6.0000) (width 0.2) (layer "F.Cu") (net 17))
 (segment (start 28.0000 6.0000) (end 43.0000 6.0000) (width 0.2) (layer "F.Cu") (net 17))
 (segment (start 13.1000 10.2700) (end 13.1000 7.2500) (width 0.2) (layer "F.Cu") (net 14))
 (segment (start 13.1000 7.2500) (end 31.0000 7.2500) (width 0.2) (layer "F.Cu") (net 14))
 (segment (start 28.0000 11.5750) (end 32.5000 11.5750) (width 0.2) (layer "F.Cu") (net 18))
 (segment (start 32.5000 11.5750) (end 32.5000 10.2500) (width 0.2) (layer "F.Cu") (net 18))
 (segment (start 13.1000 6.4600) (end 13.1000 7.7300) (width 0.2) (layer "F.Cu") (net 16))
 (segment (start 13.1000 7.7300) (end 18.9000 7.7300) (width 0.2) (layer "F.Cu") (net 16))
 (segment (start 18.9000 7.7300) (end 34.0000 7.7300) (width 0.2) (layer "F.Cu") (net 16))
 (segment (start 34.0000 7.7300) (end 34.0000 1.2500) (width 0.2) (layer "F.Cu") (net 16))
 (segment (start 31.0000 5.5750) (end 35.5000 5.5750) (width 0.2) (layer "F.Cu") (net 19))
 (segment (start 35.5000 5.5750) (end 35.5000 4.2500) (width 0.2) (layer "F.Cu") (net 19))
 (via (at 9.0000 36.0000) (size 0.8) (drill 0.4) (layers "F.Cu" "B.Cu") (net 2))
 (via (at 13.0000 36.0000) (size 0.8) (drill 0.4) (layers "F.Cu" "B.Cu") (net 2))
 (via (at 21.5750 36.9500) (size 0.8) (drill 0.4) (layers "F.Cu" "B.Cu") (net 2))
 (via (at 24.0250 32.0000) (size 0.8) (drill 0.4) (layers "F.Cu" "B.Cu") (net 2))
 (via (at 38.0250 32.0000) (size 0.8) (drill 0.4) (layers "F.Cu" "B.Cu") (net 2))
 (via (at 43.0000 32.5750) (size 0.8) (drill 0.4) (layers "F.Cu" "B.Cu") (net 2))
 (via (at 15.1100 14.3800) (size 0.8) (drill 0.4) (layers "F.Cu" "B.Cu") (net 2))
 (via (at 32.8900 16.9200) (size 0.8) (drill 0.4) (layers "F.Cu" "B.Cu") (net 2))
 (via (at 12.5750 22.0000) (size 0.8) (drill 0.4) (layers "F.Cu" "B.Cu") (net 2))
 (via (at 13.0250 18.0000) (size 0.8) (drill 0.4) (layers "F.Cu" "B.Cu") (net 2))
 (via (at 40.2500 19.6250) (size 0.8) (drill 0.4) (layers "F.Cu" "B.Cu") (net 2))
 (via (at 41.7500 19.6250) (size 0.8) (drill 0.4) (layers "F.Cu" "B.Cu") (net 2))
 (via (at 43.3750 20.7500) (size 0.8) (drill 0.4) (layers "F.Cu" "B.Cu") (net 2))
 (via (at 43.3750 21.7500) (size 0.8) (drill 0.4) (layers "F.Cu" "B.Cu") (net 2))
 (via (at 41.0000 22.0000) (size 0.8) (drill 0.4) (layers "F.Cu" "B.Cu") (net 2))
 (via (at 37.5750 22.0000) (size 0.8) (drill 0.4) (layers "F.Cu" "B.Cu") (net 2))
 (via (at 38.0250 17.0000) (size 0.8) (drill 0.4) (layers "F.Cu" "B.Cu") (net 2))
 (via (at 45.5750 17.0000) (size 0.8) (drill 0.4) (layers "F.Cu" "B.Cu") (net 2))
 (via (at 18.9000 5.1900) (size 0.8) (drill 0.4) (layers "F.Cu" "B.Cu") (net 2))
 (via (at 8.5750 12.0000) (size 0.8) (drill 0.4) (layers "F.Cu" "B.Cu") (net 2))
 (via (at 9.0250 8.0000) (size 0.8) (drill 0.4) (layers "F.Cu" "B.Cu") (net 2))
 (via (at 29.5000 10.2500) (size 0.8) (drill 0.4) (layers "F.Cu" "B.Cu") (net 2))
 (via (at 41.0000 6.0000) (size 0.8) (drill 0.4) (layers "F.Cu" "B.Cu") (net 2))
 (via (at 32.5000 4.2500) (size 0.8) (drill 0.4) (layers "F.Cu" "B.Cu") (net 2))
 (via (at 45.0000 12.0000) (size 0.8) (drill 0.4) (layers "F.Cu" "B.Cu") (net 2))
 (via (at 45.0000 6.0000) (size 0.8) (drill 0.4) (layers "F.Cu" "B.Cu") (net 2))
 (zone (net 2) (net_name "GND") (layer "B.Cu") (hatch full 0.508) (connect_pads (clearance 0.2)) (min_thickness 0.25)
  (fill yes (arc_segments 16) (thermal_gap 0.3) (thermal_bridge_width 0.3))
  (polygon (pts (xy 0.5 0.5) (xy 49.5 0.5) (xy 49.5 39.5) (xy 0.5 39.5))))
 (gr_line (start 0 0) (end 50.0 0) (stroke (width 0.05) (type default)) (layer "Edge.Cuts"))
 (gr_line (start 50.0 0) (end 50.0 40.0) (stroke (width 0.05) (type default)) (layer "Edge.Cuts"))
 (gr_line (start 50.0 40.0) (end 0 40.0) (stroke (width 0.05) (type default)) (layer "Edge.Cuts"))
 (gr_line (start 0 40.0) (end 0 0) (stroke (width 0.05) (type default)) (layer "Edge.Cuts")))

